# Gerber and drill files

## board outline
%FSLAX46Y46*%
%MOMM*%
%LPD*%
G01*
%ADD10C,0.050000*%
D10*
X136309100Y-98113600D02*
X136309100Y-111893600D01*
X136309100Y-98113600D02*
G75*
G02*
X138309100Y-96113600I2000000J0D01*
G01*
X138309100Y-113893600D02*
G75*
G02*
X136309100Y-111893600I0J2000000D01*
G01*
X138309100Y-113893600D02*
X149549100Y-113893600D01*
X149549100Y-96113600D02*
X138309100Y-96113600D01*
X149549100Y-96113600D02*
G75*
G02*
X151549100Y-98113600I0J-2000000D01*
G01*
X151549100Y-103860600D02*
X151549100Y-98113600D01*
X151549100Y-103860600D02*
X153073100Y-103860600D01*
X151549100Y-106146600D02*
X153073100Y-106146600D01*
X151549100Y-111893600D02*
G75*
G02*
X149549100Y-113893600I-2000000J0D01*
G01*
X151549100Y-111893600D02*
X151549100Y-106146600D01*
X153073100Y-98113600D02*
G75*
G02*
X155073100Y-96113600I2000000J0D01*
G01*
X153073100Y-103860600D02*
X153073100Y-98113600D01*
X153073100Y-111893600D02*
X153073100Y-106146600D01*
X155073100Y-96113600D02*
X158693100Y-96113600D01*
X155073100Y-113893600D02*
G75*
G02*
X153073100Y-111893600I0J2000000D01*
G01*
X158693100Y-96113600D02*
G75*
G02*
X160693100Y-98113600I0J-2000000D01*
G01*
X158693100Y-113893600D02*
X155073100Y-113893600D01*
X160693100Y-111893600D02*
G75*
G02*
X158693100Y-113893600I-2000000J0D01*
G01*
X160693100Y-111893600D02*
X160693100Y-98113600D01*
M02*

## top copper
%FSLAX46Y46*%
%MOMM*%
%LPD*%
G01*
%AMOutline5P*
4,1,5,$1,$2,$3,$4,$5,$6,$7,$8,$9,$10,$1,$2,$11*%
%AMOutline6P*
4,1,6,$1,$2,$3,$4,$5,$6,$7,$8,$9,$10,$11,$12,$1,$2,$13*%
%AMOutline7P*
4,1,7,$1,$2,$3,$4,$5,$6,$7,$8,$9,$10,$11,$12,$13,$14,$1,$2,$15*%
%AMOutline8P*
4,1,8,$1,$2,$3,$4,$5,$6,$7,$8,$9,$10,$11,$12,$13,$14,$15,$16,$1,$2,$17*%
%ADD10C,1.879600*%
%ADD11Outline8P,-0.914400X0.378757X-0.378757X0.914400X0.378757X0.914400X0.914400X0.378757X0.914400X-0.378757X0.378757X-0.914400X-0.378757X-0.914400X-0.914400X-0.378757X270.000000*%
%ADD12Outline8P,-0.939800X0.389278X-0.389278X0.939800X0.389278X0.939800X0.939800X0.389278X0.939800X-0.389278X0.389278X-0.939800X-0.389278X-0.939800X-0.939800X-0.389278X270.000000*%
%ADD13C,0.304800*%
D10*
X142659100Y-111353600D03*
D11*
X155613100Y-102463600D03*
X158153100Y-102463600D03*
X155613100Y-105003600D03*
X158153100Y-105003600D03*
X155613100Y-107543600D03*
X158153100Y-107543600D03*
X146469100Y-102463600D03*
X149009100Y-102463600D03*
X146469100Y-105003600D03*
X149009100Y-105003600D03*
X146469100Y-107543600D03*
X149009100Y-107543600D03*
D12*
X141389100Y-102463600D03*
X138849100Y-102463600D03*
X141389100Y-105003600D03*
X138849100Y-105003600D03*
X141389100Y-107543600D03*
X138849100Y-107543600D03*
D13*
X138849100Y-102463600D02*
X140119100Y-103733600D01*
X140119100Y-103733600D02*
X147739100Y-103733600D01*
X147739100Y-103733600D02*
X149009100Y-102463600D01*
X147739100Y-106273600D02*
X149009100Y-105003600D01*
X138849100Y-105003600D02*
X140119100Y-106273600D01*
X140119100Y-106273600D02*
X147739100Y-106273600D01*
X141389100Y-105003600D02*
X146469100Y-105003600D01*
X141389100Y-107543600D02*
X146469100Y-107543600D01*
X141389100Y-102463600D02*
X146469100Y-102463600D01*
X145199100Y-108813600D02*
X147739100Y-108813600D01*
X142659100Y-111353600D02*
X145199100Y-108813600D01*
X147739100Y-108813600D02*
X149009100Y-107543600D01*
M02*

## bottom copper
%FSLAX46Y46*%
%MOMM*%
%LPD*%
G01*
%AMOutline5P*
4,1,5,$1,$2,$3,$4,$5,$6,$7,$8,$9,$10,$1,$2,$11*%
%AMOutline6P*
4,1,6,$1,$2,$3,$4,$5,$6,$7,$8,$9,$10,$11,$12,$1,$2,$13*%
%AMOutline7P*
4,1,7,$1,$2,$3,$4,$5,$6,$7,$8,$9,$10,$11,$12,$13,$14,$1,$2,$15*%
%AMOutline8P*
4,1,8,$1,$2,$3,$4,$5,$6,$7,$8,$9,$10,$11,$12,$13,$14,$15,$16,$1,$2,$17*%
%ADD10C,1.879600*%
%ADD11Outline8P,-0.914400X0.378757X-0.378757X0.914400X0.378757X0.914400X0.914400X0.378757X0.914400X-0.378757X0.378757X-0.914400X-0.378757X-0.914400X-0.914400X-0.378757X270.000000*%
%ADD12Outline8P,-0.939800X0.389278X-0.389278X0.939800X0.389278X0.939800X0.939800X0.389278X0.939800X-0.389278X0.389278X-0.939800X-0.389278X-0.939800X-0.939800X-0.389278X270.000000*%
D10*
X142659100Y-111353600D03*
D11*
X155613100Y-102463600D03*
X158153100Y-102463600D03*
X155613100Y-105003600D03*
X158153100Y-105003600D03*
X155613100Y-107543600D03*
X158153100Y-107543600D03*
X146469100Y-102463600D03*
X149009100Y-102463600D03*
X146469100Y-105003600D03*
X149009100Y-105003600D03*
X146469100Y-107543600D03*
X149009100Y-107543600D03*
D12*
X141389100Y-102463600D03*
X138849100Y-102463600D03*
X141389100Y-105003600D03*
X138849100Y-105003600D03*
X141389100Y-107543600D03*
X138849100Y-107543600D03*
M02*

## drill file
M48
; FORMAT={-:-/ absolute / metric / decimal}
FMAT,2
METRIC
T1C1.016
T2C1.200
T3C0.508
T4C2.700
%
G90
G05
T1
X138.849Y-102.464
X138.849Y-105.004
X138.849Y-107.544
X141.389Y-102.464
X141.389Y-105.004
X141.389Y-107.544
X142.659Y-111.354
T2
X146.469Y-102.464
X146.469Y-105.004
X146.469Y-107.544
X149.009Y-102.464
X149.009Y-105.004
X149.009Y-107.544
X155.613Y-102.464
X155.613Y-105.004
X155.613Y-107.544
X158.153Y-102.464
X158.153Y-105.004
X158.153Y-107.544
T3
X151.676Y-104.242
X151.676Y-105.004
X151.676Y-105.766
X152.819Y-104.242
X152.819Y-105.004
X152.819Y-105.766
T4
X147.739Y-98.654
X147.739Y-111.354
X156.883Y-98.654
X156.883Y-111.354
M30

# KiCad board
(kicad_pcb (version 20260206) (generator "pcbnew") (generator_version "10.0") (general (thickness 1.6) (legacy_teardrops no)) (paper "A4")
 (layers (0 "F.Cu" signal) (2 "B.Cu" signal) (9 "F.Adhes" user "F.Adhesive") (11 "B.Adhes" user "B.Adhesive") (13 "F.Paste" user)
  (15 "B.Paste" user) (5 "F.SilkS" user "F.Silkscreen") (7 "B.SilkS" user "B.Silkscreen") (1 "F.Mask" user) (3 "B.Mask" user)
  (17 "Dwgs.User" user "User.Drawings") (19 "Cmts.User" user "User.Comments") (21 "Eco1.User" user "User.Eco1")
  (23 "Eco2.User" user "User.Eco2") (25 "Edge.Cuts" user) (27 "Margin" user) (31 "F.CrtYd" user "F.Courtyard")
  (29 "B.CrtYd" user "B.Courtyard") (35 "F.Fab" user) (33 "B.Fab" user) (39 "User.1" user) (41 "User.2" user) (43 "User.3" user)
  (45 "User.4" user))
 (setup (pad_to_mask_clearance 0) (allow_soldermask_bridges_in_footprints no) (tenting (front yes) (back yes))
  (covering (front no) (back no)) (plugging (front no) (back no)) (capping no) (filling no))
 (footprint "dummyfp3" (layer "F.Cu") (at 156.8831 111.3536)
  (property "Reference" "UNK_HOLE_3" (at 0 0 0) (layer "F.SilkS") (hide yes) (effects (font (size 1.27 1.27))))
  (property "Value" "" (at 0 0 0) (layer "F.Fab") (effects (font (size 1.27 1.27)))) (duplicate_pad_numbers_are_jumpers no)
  (pad "" np_thru_hole circle (at 0 0) (size 2.7 2.7) (drill 2.7) (layers "*.Cu" "*.Mask")))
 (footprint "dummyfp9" (layer "F.Cu") (at 151.6761 105.7656)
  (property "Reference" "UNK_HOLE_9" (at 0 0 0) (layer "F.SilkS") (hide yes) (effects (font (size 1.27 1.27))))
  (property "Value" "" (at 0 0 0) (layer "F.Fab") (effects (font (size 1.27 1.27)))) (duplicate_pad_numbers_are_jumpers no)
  (pad "" np_thru_hole circle (at 0 0) (size 0.508 0.508) (drill 0.508) (layers "*.Cu" "*.Mask")))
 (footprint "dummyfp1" (layer "F.Cu") (at 147.7391 98.6536)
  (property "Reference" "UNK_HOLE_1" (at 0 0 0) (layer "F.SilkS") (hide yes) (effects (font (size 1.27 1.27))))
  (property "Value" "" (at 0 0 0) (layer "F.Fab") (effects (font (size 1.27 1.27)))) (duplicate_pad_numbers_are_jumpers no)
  (pad "" np_thru_hole circle (at 0 0) (size 2.7 2.7) (drill 2.7) (layers "*.Cu" "*.Mask")))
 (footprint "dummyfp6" (layer "F.Cu") (at 152.8191 105.7656)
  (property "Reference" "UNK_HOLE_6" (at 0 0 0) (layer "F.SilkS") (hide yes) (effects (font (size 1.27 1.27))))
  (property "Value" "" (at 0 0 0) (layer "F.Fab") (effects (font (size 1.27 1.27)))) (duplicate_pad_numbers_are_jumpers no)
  (pad "" np_thru_hole circle (at 0 0) (size 0.508 0.508) (drill 0.508) (layers "*.Cu" "*.Mask")))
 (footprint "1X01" (layer "F.Cu") (at 142.6591 111.3536)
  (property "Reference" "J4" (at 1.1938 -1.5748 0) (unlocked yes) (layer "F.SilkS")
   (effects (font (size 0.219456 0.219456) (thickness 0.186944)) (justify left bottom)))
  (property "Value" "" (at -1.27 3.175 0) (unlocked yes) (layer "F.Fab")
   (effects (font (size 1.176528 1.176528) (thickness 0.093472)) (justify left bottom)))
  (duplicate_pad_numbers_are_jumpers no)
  (pad "1" thru_hole circle (at 0 0 90) (size 1.8796 1.8796) (drill 1.016) (layers "*.Cu" "*.Mask") (remove_unused_layers no) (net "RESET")
   (solder_mask_margin 0.0635) (thermal_bridge_angle 0)))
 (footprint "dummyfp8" (layer "F.Cu") (at 151.6761 105.0036)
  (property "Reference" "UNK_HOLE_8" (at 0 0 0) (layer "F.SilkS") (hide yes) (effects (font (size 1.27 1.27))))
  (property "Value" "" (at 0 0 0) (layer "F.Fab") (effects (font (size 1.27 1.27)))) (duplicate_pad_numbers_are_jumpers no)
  (pad "" np_thru_hole circle (at 0 0) (size 0.508 0.508) (drill 0.508) (layers "*.Cu" "*.Mask")))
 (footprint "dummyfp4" (layer "F.Cu") (at 152.8191 104.2416)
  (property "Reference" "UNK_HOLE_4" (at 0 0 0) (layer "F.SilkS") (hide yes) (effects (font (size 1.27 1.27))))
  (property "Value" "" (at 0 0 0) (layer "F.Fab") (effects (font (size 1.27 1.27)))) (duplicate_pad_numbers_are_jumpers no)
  (pad "" np_thru_hole circle (at 0 0) (size 0.508 0.508) (drill 0.508) (layers "*.Cu" "*.Mask")))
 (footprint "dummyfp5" (layer "F.Cu") (at 152.8191 105.0036)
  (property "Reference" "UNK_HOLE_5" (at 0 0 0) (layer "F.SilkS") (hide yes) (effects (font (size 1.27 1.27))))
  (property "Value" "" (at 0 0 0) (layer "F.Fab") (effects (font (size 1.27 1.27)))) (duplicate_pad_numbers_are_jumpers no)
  (pad "" np_thru_hole circle (at 0 0) (size 0.508 0.508) (drill 0.508) (layers "*.Cu" "*.Mask")))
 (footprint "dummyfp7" (layer "F.Cu") (at 151.6761 104.2416)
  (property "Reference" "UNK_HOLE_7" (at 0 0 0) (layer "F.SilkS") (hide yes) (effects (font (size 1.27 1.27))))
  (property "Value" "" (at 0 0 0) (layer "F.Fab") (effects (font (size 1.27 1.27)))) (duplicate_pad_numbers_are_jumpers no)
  (pad "" np_thru_hole circle (at 0 0) (size 0.508 0.508) (drill 0.508) (layers "*.Cu" "*.Mask")))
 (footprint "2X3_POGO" (layer "F.Cu") (at 156.8831 105.0036 -90)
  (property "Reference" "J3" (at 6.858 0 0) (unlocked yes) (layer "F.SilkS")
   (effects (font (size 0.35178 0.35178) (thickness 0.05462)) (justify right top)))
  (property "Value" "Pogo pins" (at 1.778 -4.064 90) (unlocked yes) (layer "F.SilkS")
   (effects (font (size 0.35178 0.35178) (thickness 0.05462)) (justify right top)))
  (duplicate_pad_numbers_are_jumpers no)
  (pad "P$1" thru_hole roundrect (at -2.54 1.27 270) (size 1.8288 1.8288) (drill 1.2) (layers "*.Cu" "*.Mask") (remove_unused_layers no)
   (roundrect_rratio 0.25) (chamfer_ratio 0.2928932188) (chamfer top_left top_right bottom_left bottom_right) (solder_mask_margin 0.0635)
   (thermal_bridge_angle 0))
  (pad "P$2" thru_hole roundrect (at -2.54 -1.27 270) (size 1.8288 1.8288) (drill 1.2) (layers "*.Cu" "*.Mask") (remove_unused_layers no)
   (roundrect_rratio 0.25) (chamfer_ratio 0.2928932188) (chamfer top_left top_right bottom_left bottom_right) (solder_mask_margin 0.0635)
   (thermal_bridge_angle 0))
  (pad "P$3" thru_hole roundrect (at 0 1.27 270) (size 1.8288 1.8288) (drill 1.2) (layers "*.Cu" "*.Mask") (remove_unused_layers no)
   (roundrect_rratio 0.25) (chamfer_ratio 0.2928932188) (chamfer top_left top_right bottom_left bottom_right) (solder_mask_margin 0.0635)
   (thermal_bridge_angle 0))
  (pad "P$4" thru_hole roundrect (at 0 -1.27 270) (size 1.8288 1.8288) (drill 1.2) (layers "*.Cu" "*.Mask") (remove_unused_layers no)
   (roundrect_rratio 0.25) (chamfer_ratio 0.2928932188) (chamfer top_left top_right bottom_left bottom_right) (solder_mask_margin 0.0635)
   (thermal_bridge_angle 0))
  (pad "P$5" thru_hole roundrect (at 2.54 1.27 270) (size 1.8288 1.8288) (drill 1.2) (layers "*.Cu" "*.Mask") (remove_unused_layers no)
   (roundrect_rratio 0.25) (chamfer_ratio 0.2928932188) (chamfer top_left top_right bottom_left bottom_right) (solder_mask_margin 0.0635)
   (thermal_bridge_angle 0))
  (pad "P$6" thru_hole roundrect (at 2.54 -1.27 270) (size 1.8288 1.8288) (drill 1.2) (layers "*.Cu" "*.Mask") (remove_unused_layers no)
   (roundrect_rratio 0.25) (chamfer_ratio 0.2928932188) (chamfer top_left top_right bottom_left bottom_right) (solder_mask_margin 0.0635)
   (thermal_bridge_angle 0)))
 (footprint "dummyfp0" (layer "F.Cu") (at 147.7391 111.3536)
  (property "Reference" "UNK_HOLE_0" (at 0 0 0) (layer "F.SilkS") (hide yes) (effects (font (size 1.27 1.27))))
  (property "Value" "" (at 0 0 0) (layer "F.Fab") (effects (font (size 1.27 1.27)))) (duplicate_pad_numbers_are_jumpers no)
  (pad "" np_thru_hole circle (at 0 0) (size 2.7 2.7) (drill 2.7) (layers "*.Cu" "*.Mask")))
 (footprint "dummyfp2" (layer "F.Cu") (at 156.8831 98.6536)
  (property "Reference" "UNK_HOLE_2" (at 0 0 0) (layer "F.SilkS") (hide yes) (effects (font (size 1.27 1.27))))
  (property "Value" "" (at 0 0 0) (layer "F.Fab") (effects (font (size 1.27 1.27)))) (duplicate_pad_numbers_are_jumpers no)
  (pad "" np_thru_hole circle (at 0 0) (size 2.7 2.7) (drill 2.7) (layers "*.Cu" "*.Mask")))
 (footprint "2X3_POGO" (layer "F.Cu") (at 147.7391 105.0036 -90)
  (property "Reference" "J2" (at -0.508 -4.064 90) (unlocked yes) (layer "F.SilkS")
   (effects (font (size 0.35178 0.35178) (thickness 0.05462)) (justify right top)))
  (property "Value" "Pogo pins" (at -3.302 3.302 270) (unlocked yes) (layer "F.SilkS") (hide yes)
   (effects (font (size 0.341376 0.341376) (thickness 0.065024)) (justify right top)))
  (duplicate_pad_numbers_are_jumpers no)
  (pad "P$1" thru_hole roundrect (at -2.54 1.27 270) (size 1.8288 1.8288) (drill 1.2) (layers "*.Cu" "*.Mask") (remove_unused_layers no)
   (roundrect_rratio 0.25) (chamfer_ratio 0.2928932188) (chamfer top_left top_right bottom_left bottom_right) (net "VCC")
   (solder_mask_margin 0.0635) (thermal_bridge_angle 0))
  (pad "P$2" thru_hole roundrect (at -2.54 -1.27 270) (size 1.8288 1.8288) (drill 1.2) (layers "*.Cu" "*.Mask") (remove_unused_layers no)
   (roundrect_rratio 0.25) (chamfer_ratio 0.2928932188) (chamfer top_left top_right bottom_left bottom_right) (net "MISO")
   (solder_mask_margin 0.0635) (thermal_bridge_angle 0))
  (pad "P$3" thru_hole roundrect (at 0 1.27 270) (size 1.8288 1.8288) (drill 1.2) (layers "*.Cu" "*.Mask") (remove_unused_layers no)
   (roundrect_rratio 0.25) (chamfer_ratio 0.2928932188) (chamfer top_left top_right bottom_left bottom_right) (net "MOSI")
   (solder_mask_margin 0.0635) (thermal_bridge_angle 0))
  (pad "P$4" thru_hole roundrect (at 0 -1.27 270) (size 1.8288 1.8288) (drill 1.2) (layers "*.Cu" "*.Mask") (remove_unused_layers no)
   (roundrect_rratio 0.25) (chamfer_ratio 0.2928932188) (chamfer top_left top_right bottom_left bottom_right) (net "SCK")
   (solder_mask_margin 0.0635) (thermal_bridge_angle 0))
  (pad "P$5" thru_hole roundrect (at 2.54 1.27 270) (size 1.8288 1.8288) (drill 1.2) (layers "*.Cu" "*.Mask") (remove_unused_layers no)
   (roundrect_rratio 0.25) (chamfer_ratio 0.2928932188) (chamfer top_left top_right bottom_left bottom_right) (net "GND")
   (solder_mask_margin 0.0635) (thermal_bridge_angle 0))
  (pad "P$6" thru_hole roundrect (at 2.54 -1.27 270) (size 1.8288 1.8288) (drill 1.2) (layers "*.Cu" "*.Mask") (remove_unused_layers no)
   (roundrect_rratio 0.25) (chamfer_ratio 0.2928932188) (chamfer top_left top_right bottom_left bottom_right) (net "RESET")
   (solder_mask_margin 0.0635) (thermal_bridge_angle 0)))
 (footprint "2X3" (layer "B.Cu") (at 140.1191 105.0036 -90)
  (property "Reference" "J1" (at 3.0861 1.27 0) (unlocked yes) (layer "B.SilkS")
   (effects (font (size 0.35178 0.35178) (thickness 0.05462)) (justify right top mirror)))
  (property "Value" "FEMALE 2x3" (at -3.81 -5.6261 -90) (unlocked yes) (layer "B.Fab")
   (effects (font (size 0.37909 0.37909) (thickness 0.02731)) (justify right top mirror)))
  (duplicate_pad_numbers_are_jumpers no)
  (pad "1" thru_hole roundrect (at -2.54 -1.27 270) (size 1.8796 1.8796) (drill 1.016) (layers "*.Cu" "*.Mask") (remove_unused_layers no)
   (roundrect_rratio 0.25) (chamfer_ratio 0.2928932188) (chamfer top_left top_right bottom_left bottom_right) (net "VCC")
   (solder_mask_margin 0.0635) (thermal_bridge_angle 0))
  (pad "2" thru_hole roundrect (at -2.54 1.27 270) (size 1.8796 1.8796) (drill 1.016) (layers "*.Cu" "*.Mask") (remove_unused_layers no)
   (roundrect_rratio 0.25) (chamfer_ratio 0.2928932188) (chamfer top_left top_right bottom_left bottom_right) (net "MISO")
   (solder_mask_margin 0.0635) (thermal_bridge_angle 0))
  (pad "3" thru_hole roundrect (at 0 -1.27 270) (size 1.8796 1.8796) (drill 1.016) (layers "*.Cu" "*.Mask") (remove_unused_layers no)
   (roundrect_rratio 0.25) (chamfer_ratio 0.2928932188) (chamfer top_left top_right bottom_left bottom_right) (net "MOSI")
   (solder_mask_margin 0.0635) (thermal_bridge_angle 0))
  (pad "4" thru_hole roundrect (at 0 1.27 270) (size 1.8796 1.8796) (drill 1.016) (layers "*.Cu" "*.Mask") (remove_unused_layers no)
   (roundrect_rratio 0.25) (chamfer_ratio 0.2928932188) (chamfer top_left top_right bottom_left bottom_right) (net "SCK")
   (solder_mask_margin 0.0635) (thermal_bridge_angle 0))
  (pad "5" thru_hole roundrect (at 2.54 -1.27 270) (size 1.8796 1.8796) (drill 1.016) (layers "*.Cu" "*.Mask") (remove_unused_layers no)
   (roundrect_rratio 0.25) (chamfer_ratio 0.2928932188) (chamfer top_left top_right bottom_left bottom_right) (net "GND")
   (solder_mask_margin 0.0635) (thermal_bridge_angle 0))
  (pad "6" thru_hole roundrect (at 2.54 1.27 270) (size 1.8796 1.8796) (drill 1.016) (layers "*.Cu" "*.Mask") (remove_unused_layers no)
   (roundrect_rratio 0.25) (chamfer_ratio 0.2928932188) (chamfer top_left top_right bottom_left bottom_right) (solder_mask_margin 0.0635)
   (thermal_bridge_angle 0)))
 (gr_line (start 136.3091 98.1136) (end 136.3091 111.8936) (stroke (width 0.05) (type solid)) (layer "Edge.Cuts"))
 (gr_arc (start 136.3091 98.1136) (mid 136.894886 96.699386) (end 138.3091 96.1136) (stroke (width 0.05) (type solid)) (layer "Edge.Cuts"))
 (gr_arc (start 138.3091 113.8936) (mid 136.894886 113.307814) (end 136.3091 111.8936) (stroke (width 0.05) (type solid))
  (layer "Edge.Cuts"))
 (gr_line (start 138.3091 113.8936) (end 149.5491 113.8936) (stroke (width 0.05) (type solid)) (layer "Edge.Cuts"))
 (gr_line (start 149.5491 96.1136) (end 138.3091 96.1136) (stroke (width 0.05) (type solid)) (layer "Edge.Cuts"))
 (gr_arc (start 149.5491 96.1136) (mid 150.963314 96.699386) (end 151.5491 98.1136) (stroke (width 0.05) (type solid)) (layer "Edge.Cuts"))
 (gr_line (start 151.5491 103.8606) (end 151.5491 98.1136) (stroke (width 0.05) (type solid)) (layer "Edge.Cuts"))
 (gr_line (start 151.5491 103.8606) (end 153.0731 103.8606) (stroke (width 0.05) (type solid)) (layer "Edge.Cuts"))
 (gr_line (start 151.5491 106.1466) (end 153.0731 106.1466) (stroke (width 0.05) (type solid)) (layer "Edge.Cuts"))
 (gr_arc (start 151.5491 111.8936) (mid 150.963314 113.307814) (end 149.5491 113.8936) (stroke (width 0.05) (type solid))
  (layer "Edge.Cuts"))
 (gr_line (start 151.5491 111.8936) (end 151.5491 106.1466) (stroke (width 0.05) (type solid)) (layer "Edge.Cuts"))
 (gr_arc (start 153.0731 98.1136) (mid 153.658886 96.699386) (end 155.0731 96.1136) (stroke (width 0.05) (type solid)) (layer "Edge.Cuts"))
 (gr_line (start 153.0731 103.8606) (end 153.0731 98.1136) (stroke (width 0.05) (type solid)) (layer "Edge.Cuts"))
 (gr_line (start 153.0731 111.8936) (end 153.0731 106.1466) (stroke (width 0.05) (type solid)) (layer "Edge.Cuts"))
 (gr_line (start 155.0731 96.1136) (end 158.6931 96.1136) (stroke (width 0.05) (type solid)) (layer "Edge.Cuts"))
 (gr_arc (start 155.0731 113.8936) (mid 153.658886 113.307814) (end 153.0731 111.8936) (stroke (width 0.05) (type solid))
  (layer "Edge.Cuts"))
 (gr_arc (start 158.6931 96.1136) (mid 160.107314 96.699386) (end 160.6931 98.1136) (stroke (width 0.05) (type solid)) (layer "Edge.Cuts"))
 (gr_line (start 158.6931 113.8936) (end 155.0731 113.8936) (stroke (width 0.05) (type solid)) (layer "Edge.Cuts"))
 (gr_arc (start 160.6931 111.8936) (mid 160.107314 113.307814) (end 158.6931 113.8936) (stroke (width 0.05) (type solid))
  (layer "Edge.Cuts"))
 (gr_line (start 160.6931 111.8936) (end 160.6931 98.1136) (stroke (width 0.05) (type solid)) (layer "Edge.Cuts"))
 (segment (start 138.8491 102.4636) (end 140.1191 103.7336) (width 0.3048) (layer "F.Cu") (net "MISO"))
 (segment (start 140.1191 103.7336) (end 147.7391 103.7336) (width 0.3048) (layer "F.Cu") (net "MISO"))
 (segment (start 147.7391 103.7336) (end 149.0091 102.4636) (width 0.3048) (layer "F.Cu") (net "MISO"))
 (segment (start 147.7391 106.2736) (end 149.0091 105.0036) (width 0.3048) (layer "F.Cu") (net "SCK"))
 (segment (start 138.8491 105.0036) (end 140.1191 106.2736) (width 0.3048) (layer "F.Cu") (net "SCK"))
 (segment (start 140.1191 106.2736) (end 147.7391 106.2736) (width 0.3048) (layer "F.Cu") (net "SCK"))
 (segment (start 141.3891 105.0036) (end 146.4691 105.0036) (width 0.3048) (layer "F.Cu") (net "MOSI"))
 (segment (start 141.3891 107.5436) (end 146.4691 107.5436) (width 0.3048) (layer "F.Cu") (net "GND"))
 (segment (start 141.3891 102.4636) (end 146.4691 102.4636) (width 0.3048) (layer "F.Cu") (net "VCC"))
 (segment (start 145.1991 108.8136) (end 147.7391 108.8136) (width 0.3048) (layer "F.Cu") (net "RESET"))
 (segment (start 142.6591 111.3536) (end 145.1991 108.8136) (width 0.3048) (layer "F.Cu") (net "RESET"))
 (segment (start 147.7391 108.8136) (end 149.0091 107.5436) (width 0.3048) (layer "F.Cu") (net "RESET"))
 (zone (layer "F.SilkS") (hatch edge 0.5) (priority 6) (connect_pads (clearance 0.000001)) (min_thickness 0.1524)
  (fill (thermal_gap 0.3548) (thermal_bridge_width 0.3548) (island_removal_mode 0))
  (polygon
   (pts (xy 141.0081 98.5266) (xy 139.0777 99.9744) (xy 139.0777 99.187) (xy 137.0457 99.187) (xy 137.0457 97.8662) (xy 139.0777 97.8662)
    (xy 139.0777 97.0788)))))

